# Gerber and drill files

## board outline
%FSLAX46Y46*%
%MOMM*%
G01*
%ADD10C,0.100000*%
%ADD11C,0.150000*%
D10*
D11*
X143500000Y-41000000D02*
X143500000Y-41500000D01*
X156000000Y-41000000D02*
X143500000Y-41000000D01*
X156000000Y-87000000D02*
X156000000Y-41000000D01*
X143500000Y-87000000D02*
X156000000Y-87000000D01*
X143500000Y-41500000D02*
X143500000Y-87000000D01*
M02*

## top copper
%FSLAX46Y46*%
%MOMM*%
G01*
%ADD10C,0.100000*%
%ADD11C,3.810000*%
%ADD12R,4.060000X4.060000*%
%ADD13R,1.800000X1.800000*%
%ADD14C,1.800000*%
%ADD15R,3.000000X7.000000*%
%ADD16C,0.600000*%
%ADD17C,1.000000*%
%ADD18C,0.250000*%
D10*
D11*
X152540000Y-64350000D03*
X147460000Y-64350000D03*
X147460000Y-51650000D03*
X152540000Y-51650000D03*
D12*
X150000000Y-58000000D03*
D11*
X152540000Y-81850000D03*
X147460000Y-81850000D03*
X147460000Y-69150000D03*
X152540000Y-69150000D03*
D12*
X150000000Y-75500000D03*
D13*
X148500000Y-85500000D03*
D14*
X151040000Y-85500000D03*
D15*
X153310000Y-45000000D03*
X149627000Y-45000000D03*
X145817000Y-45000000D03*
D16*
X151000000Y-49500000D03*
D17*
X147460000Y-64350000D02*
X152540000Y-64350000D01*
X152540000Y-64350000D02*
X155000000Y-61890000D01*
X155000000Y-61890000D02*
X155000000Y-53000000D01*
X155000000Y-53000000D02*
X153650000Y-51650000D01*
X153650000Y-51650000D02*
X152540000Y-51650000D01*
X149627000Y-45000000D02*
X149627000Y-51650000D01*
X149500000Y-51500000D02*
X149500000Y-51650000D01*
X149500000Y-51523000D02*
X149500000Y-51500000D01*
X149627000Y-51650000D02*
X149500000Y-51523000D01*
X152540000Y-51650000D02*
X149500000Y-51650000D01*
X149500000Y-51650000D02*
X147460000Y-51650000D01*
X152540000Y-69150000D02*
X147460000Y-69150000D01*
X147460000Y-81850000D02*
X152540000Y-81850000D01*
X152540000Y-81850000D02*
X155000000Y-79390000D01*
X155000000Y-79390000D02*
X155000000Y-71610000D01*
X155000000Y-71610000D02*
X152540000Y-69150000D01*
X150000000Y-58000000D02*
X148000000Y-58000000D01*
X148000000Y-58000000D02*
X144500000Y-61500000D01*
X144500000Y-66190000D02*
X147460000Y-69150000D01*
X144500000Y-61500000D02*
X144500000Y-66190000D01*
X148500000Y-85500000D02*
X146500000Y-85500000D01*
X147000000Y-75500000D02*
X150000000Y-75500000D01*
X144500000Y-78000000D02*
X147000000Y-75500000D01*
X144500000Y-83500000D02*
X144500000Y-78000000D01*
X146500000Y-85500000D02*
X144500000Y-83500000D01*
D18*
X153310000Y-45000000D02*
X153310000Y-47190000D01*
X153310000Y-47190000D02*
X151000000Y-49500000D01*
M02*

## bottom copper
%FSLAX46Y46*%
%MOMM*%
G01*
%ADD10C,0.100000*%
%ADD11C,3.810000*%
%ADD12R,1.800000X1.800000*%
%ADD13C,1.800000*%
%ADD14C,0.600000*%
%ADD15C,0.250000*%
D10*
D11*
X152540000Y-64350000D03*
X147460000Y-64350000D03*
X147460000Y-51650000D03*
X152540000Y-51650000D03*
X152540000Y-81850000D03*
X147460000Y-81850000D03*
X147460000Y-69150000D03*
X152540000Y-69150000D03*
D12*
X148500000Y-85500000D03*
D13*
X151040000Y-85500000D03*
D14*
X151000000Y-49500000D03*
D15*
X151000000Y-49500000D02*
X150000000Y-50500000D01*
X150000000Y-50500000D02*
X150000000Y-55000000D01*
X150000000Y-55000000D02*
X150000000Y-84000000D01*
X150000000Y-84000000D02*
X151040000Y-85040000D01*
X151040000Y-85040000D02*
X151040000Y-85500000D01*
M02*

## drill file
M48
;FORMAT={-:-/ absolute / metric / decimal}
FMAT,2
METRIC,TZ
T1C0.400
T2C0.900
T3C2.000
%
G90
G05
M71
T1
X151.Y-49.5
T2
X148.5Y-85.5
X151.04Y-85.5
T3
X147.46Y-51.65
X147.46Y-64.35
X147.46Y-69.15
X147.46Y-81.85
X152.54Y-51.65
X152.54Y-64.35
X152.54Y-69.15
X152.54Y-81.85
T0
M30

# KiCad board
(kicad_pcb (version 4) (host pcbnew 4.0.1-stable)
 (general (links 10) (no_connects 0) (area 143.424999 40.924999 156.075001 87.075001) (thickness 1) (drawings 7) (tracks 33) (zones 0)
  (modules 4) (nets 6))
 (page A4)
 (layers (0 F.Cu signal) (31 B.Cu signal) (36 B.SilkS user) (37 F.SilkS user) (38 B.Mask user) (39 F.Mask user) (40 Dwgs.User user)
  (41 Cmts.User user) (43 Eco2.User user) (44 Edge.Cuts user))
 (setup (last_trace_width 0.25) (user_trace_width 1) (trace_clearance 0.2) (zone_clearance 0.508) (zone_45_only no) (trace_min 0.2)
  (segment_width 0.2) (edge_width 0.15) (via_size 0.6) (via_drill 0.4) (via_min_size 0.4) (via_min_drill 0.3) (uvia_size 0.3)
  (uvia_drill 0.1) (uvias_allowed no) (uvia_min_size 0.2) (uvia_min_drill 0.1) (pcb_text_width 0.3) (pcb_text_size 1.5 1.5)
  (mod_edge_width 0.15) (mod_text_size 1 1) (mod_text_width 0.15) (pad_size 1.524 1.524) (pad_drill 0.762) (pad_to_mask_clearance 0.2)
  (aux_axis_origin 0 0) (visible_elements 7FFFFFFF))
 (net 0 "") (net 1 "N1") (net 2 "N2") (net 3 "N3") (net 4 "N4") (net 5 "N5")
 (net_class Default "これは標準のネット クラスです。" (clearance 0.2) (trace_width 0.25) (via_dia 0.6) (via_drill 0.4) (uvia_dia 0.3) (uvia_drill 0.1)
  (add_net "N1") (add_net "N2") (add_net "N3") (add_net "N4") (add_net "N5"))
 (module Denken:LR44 (layer F.Cu) (at 150 58 90)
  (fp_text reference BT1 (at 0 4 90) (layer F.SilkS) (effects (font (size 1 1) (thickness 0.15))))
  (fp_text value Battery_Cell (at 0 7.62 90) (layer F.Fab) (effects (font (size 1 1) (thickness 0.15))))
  (pad 1 thru_hole circle (at -6.35 2.54 90) (size 3.81 3.81) (drill 2) (layers *.Cu *.Mask F.SilkS) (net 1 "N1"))
  (pad 1 thru_hole circle (at -6.35 -2.54 90) (size 3.81 3.81) (drill 2) (layers *.Cu *.Mask F.SilkS) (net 1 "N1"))
  (pad 1 thru_hole circle (at 6.35 -2.54 90) (size 3.81 3.81) (drill 2) (layers *.Cu *.Mask F.SilkS) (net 1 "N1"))
  (pad 1 thru_hole circle (at 6.35 2.54 90) (size 3.81 3.81) (drill 2) (layers *.Cu *.Mask F.SilkS) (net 1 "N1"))
  (pad 2 smd rect (at 0 0 90) (size 4.06 4.06) (layers F.Cu F.Mask) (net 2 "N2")))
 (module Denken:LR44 (layer F.Cu) (at 150 75.5 90)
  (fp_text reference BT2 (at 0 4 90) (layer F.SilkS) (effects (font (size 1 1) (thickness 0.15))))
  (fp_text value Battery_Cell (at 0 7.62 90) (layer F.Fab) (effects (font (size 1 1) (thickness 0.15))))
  (pad 1 thru_hole circle (at -6.35 2.54 90) (size 3.81 3.81) (drill 2) (layers *.Cu *.Mask F.SilkS) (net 2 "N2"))
  (pad 1 thru_hole circle (at -6.35 -2.54 90) (size 3.81 3.81) (drill 2) (layers *.Cu *.Mask F.SilkS) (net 2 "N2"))
  (pad 1 thru_hole circle (at 6.35 -2.54 90) (size 3.81 3.81) (drill 2) (layers *.Cu *.Mask F.SilkS) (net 2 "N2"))
  (pad 1 thru_hole circle (at 6.35 2.54 90) (size 3.81 3.81) (drill 2) (layers *.Cu *.Mask F.SilkS) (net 2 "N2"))
  (pad 2 smd rect (at 0 0 90) (size 4.06 4.06) (layers F.Cu F.Mask) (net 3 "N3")))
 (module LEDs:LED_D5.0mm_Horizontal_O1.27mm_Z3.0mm (layer F.Cu) (at 148.5 85.5)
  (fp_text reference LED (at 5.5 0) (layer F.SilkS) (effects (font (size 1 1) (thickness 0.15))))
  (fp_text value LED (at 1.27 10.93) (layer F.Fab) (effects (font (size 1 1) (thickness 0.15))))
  (pad 1 thru_hole rect (at 0 0) (size 1.8 1.8) (drill 0.9) (layers *.Cu *.Mask) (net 3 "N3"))
  (pad 2 thru_hole circle (at 2.54 0) (size 1.8 1.8) (drill 0.9) (layers *.Cu *.Mask) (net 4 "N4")))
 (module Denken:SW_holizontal (layer F.Cu) (at 149.5 45 180)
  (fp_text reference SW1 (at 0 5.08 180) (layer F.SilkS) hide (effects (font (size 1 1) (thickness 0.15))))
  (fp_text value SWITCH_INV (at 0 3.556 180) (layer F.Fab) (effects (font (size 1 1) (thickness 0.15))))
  (pad 1 smd rect (at -3.81 0 180) (size 3 7) (layers F.Cu F.Mask) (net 4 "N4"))
  (pad 2 smd rect (at -0.127 0 180) (size 3 7) (layers F.Cu F.Mask) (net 1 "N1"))
  (pad 3 smd rect (at 3.683 0 180) (size 3 7) (layers F.Cu F.Mask) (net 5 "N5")))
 (gr_line (start 143.5 41) (end 143.5 41.5) (angle 90) (layer Edge.Cuts) (width 0.15))
 (gr_line (start 156 41) (end 143.5 41) (angle 90) (layer Edge.Cuts) (width 0.15))
 (gr_line (start 156 87) (end 156 41) (angle 90) (layer Edge.Cuts) (width 0.15))
 (gr_line (start 143.5 87) (end 156 87) (angle 90) (layer Edge.Cuts) (width 0.15))
 (gr_line (start 143.5 41.5) (end 143.5 87) (angle 90) (layer Edge.Cuts) (width 0.15))
 (segment (start 147.46 64.35) (end 152.54 64.35) (width 1) (layer F.Cu) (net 1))
 (segment (start 152.54 64.35) (end 155 61.89) (width 1) (layer F.Cu) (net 1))
 (segment (start 155 61.89) (end 155 53) (width 1) (layer F.Cu) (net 1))
 (segment (start 155 53) (end 153.65 51.65) (width 1) (layer F.Cu) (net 1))
 (segment (start 153.65 51.65) (end 152.54 51.65) (width 1) (layer F.Cu) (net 1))
 (segment (start 149.627 45) (end 149.627 51.65) (width 1) (layer F.Cu) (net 1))
 (segment (start 149.5 51.5) (end 149.5 51.65) (width 1) (layer F.Cu) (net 1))
 (segment (start 149.5 51.523) (end 149.5 51.5) (width 1) (layer F.Cu) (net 1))
 (segment (start 149.627 51.65) (end 149.5 51.523) (width 1) (layer F.Cu) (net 1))
 (segment (start 152.54 51.65) (end 149.5 51.65) (width 1) (layer F.Cu) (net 1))
 (segment (start 149.5 51.65) (end 147.46 51.65) (width 1) (layer F.Cu) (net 1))
 (segment (start 152.54 69.15) (end 147.46 69.15) (width 1) (layer F.Cu) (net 2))
 (segment (start 147.46 81.85) (end 152.54 81.85) (width 1) (layer F.Cu) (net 2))
 (segment (start 152.54 81.85) (end 155 79.39) (width 1) (layer F.Cu) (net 2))
 (segment (start 155 79.39) (end 155 71.61) (width 1) (layer F.Cu) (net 2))
 (segment (start 155 71.61) (end 152.54 69.15) (width 1) (layer F.Cu) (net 2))
 (segment (start 150 58) (end 148 58) (width 1) (layer F.Cu) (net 2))
 (segment (start 148 58) (end 144.5 61.5) (width 1) (layer F.Cu) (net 2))
 (segment (start 144.5 66.19) (end 147.46 69.15) (width 1) (layer F.Cu) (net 2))
 (segment (start 144.5 61.5) (end 144.5 66.19) (width 1) (layer F.Cu) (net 2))
 (segment (start 148.5 85.5) (end 146.5 85.5) (width 1) (layer F.Cu) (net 3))
 (segment (start 147 75.5) (end 150 75.5) (width 1) (layer F.Cu) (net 3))
 (segment (start 144.5 78) (end 147 75.5) (width 1) (layer F.Cu) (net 3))
 (segment (start 144.5 83.5) (end 144.5 78) (width 1) (layer F.Cu) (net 3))
 (segment (start 146.5 85.5) (end 144.5 83.5) (width 1) (layer F.Cu) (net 3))
 (segment (start 153.31 45) (end 153.31 47.19) (width 0.25) (layer F.Cu) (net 4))
 (segment (start 153.31 47.19) (end 151 49.5) (width 0.25) (layer F.Cu) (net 4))
 (via (at 151 49.5) (size 0.6) (drill 0.4) (layers F.Cu B.Cu) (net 4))
 (segment (start 151 49.5) (end 150 50.5) (width 0.25) (layer B.Cu) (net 4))
 (segment (start 150 50.5) (end 150 55) (width 0.25) (layer B.Cu) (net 4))
 (segment (start 150 55) (end 150 84) (width 0.25) (layer B.Cu) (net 4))
 (segment (start 150 84) (end 151.04 85.04) (width 0.25) (layer B.Cu) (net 4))
 (segment (start 151.04 85.04) (end 151.04 85.5) (width 0.25) (layer B.Cu) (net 4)))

